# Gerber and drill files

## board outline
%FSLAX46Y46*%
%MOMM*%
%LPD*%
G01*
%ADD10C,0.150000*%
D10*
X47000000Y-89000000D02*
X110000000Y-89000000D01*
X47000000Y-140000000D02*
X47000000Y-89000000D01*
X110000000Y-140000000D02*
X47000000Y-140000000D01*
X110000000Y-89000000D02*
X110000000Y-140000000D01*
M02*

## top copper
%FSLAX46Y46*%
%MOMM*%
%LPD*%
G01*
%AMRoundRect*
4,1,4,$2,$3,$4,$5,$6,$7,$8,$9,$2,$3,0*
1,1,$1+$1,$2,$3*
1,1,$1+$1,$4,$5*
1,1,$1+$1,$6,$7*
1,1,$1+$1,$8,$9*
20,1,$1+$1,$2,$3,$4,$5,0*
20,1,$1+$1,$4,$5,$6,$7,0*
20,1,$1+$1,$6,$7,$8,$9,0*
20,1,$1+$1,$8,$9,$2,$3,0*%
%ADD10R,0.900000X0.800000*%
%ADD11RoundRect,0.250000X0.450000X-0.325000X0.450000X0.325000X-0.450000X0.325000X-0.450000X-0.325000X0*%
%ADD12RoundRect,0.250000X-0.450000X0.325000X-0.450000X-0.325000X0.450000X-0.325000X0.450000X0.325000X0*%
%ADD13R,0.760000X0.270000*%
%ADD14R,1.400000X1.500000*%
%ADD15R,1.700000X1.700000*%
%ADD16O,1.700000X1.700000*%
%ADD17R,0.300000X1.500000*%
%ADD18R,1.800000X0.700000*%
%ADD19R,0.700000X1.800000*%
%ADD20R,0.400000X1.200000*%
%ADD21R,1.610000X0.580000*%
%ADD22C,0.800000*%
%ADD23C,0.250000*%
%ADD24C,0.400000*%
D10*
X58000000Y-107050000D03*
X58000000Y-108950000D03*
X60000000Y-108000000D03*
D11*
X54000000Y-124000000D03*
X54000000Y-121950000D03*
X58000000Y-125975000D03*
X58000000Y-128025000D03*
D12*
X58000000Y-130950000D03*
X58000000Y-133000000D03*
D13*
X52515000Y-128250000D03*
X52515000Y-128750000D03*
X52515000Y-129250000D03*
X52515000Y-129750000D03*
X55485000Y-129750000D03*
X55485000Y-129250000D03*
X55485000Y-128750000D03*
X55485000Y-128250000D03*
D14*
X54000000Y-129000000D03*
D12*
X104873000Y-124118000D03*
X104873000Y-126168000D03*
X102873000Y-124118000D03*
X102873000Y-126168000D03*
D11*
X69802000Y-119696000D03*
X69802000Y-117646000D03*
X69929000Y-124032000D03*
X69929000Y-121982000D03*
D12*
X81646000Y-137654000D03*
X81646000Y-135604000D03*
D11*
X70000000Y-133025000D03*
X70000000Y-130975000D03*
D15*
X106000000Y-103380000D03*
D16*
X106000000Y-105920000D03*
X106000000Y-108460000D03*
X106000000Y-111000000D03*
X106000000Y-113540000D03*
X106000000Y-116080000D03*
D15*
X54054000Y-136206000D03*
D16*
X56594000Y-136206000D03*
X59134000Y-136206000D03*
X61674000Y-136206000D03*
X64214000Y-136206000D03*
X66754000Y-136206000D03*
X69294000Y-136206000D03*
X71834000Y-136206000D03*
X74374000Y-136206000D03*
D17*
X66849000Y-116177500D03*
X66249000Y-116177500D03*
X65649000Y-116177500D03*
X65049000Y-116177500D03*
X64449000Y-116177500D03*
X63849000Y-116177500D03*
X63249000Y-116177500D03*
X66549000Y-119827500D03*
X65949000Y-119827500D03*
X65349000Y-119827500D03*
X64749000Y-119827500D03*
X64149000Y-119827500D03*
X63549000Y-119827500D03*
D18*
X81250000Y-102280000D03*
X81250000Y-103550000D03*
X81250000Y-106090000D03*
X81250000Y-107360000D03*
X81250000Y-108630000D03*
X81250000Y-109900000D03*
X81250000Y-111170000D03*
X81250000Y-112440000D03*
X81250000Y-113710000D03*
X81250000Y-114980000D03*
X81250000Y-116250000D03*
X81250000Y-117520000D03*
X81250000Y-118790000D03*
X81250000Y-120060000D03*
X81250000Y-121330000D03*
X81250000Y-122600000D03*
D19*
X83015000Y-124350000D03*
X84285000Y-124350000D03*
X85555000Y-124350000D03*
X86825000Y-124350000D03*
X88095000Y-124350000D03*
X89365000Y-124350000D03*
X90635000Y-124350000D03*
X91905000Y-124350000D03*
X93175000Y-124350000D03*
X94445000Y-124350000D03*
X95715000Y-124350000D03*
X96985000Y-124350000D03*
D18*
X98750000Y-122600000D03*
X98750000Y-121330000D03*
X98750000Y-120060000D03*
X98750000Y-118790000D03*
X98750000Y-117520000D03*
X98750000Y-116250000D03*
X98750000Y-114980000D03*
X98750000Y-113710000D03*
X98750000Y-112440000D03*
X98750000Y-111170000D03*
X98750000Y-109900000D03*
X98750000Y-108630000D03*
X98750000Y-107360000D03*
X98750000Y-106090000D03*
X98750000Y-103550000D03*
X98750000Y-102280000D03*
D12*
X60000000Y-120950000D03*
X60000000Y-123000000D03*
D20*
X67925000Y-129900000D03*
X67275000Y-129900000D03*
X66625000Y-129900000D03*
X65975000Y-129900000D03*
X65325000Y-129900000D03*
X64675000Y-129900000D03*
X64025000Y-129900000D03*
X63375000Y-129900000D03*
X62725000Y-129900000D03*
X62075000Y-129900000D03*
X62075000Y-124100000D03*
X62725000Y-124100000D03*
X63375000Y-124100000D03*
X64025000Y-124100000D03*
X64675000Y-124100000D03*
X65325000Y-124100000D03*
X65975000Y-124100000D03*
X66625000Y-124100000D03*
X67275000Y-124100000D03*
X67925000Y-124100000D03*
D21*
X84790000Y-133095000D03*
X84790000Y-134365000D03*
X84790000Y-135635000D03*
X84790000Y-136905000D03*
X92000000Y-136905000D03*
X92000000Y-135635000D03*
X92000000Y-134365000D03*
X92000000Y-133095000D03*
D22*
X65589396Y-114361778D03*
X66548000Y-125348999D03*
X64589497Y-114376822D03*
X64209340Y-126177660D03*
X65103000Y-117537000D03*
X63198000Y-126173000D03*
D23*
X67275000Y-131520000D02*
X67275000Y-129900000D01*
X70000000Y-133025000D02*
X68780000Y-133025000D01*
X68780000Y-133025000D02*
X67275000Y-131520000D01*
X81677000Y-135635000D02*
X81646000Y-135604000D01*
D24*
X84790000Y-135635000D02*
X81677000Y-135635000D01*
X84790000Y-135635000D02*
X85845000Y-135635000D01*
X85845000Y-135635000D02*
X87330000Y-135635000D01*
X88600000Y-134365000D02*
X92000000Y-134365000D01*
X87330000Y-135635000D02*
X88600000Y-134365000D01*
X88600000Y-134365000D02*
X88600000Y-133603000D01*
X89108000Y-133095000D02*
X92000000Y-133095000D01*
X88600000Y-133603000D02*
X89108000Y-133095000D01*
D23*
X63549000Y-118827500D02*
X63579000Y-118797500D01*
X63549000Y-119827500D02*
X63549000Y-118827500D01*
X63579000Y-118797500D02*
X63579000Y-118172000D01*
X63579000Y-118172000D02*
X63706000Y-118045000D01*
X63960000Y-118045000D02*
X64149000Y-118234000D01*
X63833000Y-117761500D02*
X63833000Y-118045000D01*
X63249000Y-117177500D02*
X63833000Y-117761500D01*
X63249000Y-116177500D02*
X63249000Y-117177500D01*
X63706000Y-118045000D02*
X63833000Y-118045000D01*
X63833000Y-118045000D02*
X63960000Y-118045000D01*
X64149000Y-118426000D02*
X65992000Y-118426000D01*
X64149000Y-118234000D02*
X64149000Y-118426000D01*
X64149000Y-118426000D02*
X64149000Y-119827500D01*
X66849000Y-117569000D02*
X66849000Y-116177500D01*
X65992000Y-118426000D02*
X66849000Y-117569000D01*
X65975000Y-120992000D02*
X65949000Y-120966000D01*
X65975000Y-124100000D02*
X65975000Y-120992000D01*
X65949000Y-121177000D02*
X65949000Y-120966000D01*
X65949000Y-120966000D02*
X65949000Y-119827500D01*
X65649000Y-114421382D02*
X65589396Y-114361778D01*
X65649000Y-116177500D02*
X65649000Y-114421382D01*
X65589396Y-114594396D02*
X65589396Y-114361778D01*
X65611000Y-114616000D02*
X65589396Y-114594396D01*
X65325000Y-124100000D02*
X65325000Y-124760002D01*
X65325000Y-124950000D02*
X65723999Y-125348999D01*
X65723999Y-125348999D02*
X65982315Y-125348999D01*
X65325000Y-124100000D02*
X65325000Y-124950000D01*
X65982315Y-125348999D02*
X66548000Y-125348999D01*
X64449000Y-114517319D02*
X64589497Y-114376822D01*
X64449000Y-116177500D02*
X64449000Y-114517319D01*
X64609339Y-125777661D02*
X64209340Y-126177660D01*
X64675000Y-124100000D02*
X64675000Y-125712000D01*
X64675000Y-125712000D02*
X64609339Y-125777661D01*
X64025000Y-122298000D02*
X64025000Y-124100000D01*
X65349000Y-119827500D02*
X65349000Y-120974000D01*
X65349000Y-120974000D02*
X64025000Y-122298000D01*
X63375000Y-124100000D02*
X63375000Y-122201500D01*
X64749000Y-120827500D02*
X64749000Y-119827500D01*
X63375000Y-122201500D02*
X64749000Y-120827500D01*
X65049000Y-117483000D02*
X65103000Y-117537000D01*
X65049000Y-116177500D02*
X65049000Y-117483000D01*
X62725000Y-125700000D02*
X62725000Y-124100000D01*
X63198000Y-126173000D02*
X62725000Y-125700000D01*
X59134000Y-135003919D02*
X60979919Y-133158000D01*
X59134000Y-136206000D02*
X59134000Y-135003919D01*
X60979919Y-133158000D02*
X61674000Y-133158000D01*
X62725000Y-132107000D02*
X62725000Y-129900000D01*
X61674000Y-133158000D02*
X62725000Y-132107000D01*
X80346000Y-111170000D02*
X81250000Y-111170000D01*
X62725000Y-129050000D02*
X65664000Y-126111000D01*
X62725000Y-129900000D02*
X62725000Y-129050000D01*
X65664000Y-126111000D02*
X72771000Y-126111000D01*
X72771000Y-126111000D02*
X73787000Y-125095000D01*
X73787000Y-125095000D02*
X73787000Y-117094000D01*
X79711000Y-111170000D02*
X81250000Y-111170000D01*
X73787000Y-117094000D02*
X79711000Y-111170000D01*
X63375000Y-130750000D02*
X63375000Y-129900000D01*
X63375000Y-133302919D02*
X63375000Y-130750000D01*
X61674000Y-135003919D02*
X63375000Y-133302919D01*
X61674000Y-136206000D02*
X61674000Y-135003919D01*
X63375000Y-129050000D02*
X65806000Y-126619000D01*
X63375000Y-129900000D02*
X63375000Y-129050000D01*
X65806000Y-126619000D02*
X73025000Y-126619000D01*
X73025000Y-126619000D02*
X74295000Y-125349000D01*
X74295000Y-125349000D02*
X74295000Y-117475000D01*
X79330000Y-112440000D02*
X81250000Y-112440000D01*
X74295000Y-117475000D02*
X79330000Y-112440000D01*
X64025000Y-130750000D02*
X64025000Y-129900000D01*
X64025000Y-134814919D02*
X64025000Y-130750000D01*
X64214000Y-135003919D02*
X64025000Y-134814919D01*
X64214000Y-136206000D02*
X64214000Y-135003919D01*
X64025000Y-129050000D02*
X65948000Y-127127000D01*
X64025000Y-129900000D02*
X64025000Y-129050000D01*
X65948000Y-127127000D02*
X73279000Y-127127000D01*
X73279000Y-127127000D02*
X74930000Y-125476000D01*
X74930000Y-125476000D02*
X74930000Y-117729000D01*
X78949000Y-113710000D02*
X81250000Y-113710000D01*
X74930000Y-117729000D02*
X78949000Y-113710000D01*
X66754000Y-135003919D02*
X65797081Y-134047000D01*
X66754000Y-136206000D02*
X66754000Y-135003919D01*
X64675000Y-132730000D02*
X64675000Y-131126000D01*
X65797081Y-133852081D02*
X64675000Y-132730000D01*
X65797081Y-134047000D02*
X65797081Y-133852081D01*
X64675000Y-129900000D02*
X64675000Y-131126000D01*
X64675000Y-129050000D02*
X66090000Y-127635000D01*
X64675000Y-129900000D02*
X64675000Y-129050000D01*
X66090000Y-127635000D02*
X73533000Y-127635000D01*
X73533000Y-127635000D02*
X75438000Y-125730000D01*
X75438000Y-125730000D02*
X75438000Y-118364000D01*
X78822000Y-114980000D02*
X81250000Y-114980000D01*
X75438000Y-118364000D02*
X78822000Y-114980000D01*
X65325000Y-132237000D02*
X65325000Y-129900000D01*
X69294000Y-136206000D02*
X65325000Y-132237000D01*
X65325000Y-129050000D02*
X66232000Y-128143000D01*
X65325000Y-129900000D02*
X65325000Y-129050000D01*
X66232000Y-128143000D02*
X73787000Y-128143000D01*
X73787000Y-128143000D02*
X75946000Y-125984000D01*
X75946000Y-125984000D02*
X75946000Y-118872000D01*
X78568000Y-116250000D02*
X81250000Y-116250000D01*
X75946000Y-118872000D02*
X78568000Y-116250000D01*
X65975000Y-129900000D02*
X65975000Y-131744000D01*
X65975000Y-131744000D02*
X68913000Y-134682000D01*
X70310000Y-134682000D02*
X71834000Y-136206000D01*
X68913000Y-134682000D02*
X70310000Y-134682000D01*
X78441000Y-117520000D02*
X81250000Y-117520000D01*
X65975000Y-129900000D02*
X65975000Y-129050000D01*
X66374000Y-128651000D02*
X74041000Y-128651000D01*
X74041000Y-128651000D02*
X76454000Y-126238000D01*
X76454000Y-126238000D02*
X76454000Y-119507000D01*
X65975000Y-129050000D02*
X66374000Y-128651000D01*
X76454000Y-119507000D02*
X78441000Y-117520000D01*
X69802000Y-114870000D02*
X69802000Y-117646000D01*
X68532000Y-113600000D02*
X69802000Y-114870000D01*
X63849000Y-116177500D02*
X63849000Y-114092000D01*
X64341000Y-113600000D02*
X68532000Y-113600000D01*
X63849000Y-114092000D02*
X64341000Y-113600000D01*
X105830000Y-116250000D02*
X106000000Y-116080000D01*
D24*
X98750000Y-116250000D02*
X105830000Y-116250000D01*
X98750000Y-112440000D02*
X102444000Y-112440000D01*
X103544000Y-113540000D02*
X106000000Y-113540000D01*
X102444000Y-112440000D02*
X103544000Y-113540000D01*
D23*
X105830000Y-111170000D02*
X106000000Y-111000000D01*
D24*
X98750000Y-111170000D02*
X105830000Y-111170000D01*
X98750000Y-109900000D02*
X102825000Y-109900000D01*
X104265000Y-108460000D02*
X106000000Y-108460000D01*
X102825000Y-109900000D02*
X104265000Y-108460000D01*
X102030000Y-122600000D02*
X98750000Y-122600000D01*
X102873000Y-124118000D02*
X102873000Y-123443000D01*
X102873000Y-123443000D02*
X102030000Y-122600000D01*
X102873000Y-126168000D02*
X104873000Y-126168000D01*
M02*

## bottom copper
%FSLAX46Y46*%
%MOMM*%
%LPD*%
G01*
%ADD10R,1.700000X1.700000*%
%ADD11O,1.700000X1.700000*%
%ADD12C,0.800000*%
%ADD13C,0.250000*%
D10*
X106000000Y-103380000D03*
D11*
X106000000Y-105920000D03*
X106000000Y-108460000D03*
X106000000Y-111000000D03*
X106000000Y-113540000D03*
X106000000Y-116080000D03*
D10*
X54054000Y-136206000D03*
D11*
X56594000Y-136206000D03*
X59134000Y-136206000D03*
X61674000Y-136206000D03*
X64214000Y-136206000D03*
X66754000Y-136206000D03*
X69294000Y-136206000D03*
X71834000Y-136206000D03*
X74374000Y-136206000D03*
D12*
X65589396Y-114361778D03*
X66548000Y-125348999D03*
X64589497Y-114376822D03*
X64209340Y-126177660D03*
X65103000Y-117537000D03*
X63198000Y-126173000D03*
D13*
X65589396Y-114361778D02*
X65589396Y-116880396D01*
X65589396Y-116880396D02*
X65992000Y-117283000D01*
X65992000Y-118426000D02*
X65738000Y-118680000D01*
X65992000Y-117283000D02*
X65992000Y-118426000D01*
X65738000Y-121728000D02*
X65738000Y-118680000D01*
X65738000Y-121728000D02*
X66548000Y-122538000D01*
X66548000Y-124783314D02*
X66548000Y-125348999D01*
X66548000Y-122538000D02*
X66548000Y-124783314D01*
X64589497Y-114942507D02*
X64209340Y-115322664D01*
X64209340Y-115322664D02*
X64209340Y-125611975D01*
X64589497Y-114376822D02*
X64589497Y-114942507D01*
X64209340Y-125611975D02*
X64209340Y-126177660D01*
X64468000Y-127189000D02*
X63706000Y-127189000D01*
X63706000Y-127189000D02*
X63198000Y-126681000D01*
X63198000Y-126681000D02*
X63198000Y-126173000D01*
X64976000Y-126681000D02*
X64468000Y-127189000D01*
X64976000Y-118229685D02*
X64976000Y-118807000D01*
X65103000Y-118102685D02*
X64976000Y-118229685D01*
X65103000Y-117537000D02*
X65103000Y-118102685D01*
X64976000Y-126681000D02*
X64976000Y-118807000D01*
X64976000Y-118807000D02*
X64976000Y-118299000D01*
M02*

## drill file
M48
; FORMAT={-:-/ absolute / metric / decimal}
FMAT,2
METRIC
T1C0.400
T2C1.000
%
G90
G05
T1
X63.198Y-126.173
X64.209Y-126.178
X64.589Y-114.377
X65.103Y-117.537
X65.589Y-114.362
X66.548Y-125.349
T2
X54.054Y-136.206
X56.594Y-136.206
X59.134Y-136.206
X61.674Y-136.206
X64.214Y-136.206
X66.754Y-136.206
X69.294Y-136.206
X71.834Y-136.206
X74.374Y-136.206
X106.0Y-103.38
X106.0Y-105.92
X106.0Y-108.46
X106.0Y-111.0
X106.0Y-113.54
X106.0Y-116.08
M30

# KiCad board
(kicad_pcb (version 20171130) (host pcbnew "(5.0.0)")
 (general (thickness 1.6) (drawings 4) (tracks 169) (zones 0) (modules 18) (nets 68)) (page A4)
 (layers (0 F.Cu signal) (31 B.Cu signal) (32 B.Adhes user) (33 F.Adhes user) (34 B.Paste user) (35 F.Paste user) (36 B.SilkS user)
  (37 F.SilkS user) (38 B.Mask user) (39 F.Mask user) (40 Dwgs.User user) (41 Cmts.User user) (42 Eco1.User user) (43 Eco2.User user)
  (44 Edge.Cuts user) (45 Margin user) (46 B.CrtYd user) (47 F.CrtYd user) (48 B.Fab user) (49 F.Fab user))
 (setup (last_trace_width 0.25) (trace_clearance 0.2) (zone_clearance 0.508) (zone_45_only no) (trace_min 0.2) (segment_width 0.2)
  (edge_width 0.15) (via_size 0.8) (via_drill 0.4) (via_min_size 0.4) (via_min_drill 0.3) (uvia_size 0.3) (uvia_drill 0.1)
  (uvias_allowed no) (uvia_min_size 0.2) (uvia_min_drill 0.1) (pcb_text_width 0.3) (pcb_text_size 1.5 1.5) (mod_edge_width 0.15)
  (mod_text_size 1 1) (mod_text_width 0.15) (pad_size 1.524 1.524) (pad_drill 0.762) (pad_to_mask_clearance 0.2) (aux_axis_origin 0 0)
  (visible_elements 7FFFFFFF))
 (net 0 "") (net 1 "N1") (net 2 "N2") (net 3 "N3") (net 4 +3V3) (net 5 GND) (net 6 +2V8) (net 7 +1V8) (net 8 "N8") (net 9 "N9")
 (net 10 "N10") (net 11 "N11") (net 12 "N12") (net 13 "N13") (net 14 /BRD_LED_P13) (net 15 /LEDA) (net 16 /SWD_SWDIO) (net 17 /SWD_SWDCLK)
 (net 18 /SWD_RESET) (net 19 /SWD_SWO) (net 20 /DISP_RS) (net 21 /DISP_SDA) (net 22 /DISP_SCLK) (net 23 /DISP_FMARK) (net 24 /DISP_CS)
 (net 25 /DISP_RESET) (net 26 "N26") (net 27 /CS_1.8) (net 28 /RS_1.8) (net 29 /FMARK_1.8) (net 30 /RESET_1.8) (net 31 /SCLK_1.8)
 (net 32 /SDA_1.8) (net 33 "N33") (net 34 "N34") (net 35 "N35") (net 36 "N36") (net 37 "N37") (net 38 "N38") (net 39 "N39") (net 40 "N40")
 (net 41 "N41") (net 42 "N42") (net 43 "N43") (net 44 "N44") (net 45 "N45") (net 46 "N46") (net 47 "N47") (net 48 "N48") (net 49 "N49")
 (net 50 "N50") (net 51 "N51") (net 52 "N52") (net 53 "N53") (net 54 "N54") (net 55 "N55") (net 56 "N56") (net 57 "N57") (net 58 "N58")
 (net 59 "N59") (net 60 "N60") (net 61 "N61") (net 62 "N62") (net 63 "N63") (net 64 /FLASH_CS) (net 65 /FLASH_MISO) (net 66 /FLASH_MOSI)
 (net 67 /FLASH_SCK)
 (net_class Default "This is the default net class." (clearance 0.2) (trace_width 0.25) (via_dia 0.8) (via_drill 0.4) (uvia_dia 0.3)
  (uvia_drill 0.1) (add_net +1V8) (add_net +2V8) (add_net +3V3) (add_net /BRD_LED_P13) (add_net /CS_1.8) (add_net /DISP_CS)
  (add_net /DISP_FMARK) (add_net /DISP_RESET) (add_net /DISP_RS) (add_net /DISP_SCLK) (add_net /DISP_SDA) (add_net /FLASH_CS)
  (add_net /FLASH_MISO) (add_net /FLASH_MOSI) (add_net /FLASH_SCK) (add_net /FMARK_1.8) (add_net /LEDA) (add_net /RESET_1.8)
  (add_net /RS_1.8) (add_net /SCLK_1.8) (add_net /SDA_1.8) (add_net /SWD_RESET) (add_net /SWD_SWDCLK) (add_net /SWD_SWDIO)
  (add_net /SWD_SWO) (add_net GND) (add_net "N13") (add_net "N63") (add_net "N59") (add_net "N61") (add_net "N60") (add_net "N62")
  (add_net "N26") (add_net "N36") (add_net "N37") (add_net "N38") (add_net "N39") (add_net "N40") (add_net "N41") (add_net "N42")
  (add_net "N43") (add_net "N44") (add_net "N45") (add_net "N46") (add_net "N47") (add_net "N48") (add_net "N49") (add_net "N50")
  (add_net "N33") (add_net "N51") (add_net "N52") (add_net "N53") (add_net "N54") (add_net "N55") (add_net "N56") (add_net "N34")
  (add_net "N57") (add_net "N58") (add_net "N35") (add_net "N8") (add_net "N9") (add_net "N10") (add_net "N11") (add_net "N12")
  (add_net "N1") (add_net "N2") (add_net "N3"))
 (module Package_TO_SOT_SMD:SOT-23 (layer F.Cu) (at 59 108)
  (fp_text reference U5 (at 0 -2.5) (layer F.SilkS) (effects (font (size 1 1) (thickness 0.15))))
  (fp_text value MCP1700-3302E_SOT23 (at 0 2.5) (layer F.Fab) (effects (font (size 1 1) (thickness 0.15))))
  (pad 1 smd rect (at -1 -0.95) (size 0.9 0.8) (layers F.Cu F.Paste F.Mask) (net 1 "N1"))
  (pad 2 smd rect (at -1 0.95) (size 0.9 0.8) (layers F.Cu F.Paste F.Mask) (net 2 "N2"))
  (pad 3 smd rect (at 1 0) (size 0.9 0.8) (layers F.Cu F.Paste F.Mask) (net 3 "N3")))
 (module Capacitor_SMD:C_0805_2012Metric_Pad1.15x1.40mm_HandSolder (layer F.Cu) (at 54 122.975 90)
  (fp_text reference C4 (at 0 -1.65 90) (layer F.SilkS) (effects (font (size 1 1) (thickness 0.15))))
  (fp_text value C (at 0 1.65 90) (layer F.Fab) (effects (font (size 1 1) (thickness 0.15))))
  (pad 1 smd roundrect (at -1.025 0 90) (size 1.15 1.4) (layers F.Cu F.Paste F.Mask) (roundrect_rratio 0.217391) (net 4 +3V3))
  (pad 2 smd roundrect (at 1.025 0 90) (size 1.15 1.4) (layers F.Cu F.Paste F.Mask) (roundrect_rratio 0.217391) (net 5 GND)))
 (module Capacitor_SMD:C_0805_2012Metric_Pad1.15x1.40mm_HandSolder (layer F.Cu) (at 58 127 90)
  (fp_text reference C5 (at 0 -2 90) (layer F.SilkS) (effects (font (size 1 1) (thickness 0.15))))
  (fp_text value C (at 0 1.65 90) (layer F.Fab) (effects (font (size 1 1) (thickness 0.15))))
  (pad 2 smd roundrect (at 1.025 0 90) (size 1.15 1.4) (layers F.Cu F.Paste F.Mask) (roundrect_rratio 0.217391) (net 5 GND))
  (pad 1 smd roundrect (at -1.025 0 90) (size 1.15 1.4) (layers F.Cu F.Paste F.Mask) (roundrect_rratio 0.217391) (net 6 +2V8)))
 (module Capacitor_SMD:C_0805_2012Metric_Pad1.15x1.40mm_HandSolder (layer F.Cu) (at 58 131.975 270)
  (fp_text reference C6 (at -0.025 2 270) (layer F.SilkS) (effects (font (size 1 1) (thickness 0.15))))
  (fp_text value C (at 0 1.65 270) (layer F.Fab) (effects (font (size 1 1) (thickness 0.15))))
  (pad 1 smd roundrect (at -1.025 0 270) (size 1.15 1.4) (layers F.Cu F.Paste F.Mask) (roundrect_rratio 0.217391) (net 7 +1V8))
  (pad 2 smd roundrect (at 1.025 0 270) (size 1.15 1.4) (layers F.Cu F.Paste F.Mask) (roundrect_rratio 0.217391) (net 5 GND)))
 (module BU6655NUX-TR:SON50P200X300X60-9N (layer F.Cu) (at 54 129)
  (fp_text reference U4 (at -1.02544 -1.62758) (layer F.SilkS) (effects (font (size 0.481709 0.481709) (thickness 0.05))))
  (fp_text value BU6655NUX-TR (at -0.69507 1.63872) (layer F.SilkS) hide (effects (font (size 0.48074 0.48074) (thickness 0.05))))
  (pad 1 smd rect (at -1.485 -0.75) (size 0.76 0.27) (layers F.Cu F.Paste F.Mask) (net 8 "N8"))
  (pad 2 smd rect (at -1.485 -0.25) (size 0.76 0.27) (layers F.Cu F.Paste F.Mask) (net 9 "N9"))
  (pad 3 smd rect (at -1.485 0.25) (size 0.76 0.27) (layers F.Cu F.Paste F.Mask) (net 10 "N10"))
  (pad 4 smd rect (at -1.485 0.75) (size 0.76 0.27) (layers F.Cu F.Paste F.Mask) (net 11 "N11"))
  (pad 5 smd rect (at 1.485 0.75) (size 0.76 0.27) (layers F.Cu F.Paste F.Mask) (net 5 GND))
  (pad 6 smd rect (at 1.485 0.25) (size 0.76 0.27) (layers F.Cu F.Paste F.Mask) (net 7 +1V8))
  (pad 7 smd rect (at 1.485 -0.25) (size 0.76 0.27) (layers F.Cu F.Paste F.Mask) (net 6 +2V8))
  (pad 8 smd rect (at 1.485 -0.75) (size 0.76 0.27) (layers F.Cu F.Paste F.Mask) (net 4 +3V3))
  (pad 9 smd rect (at 0 0) (size 1.4 1.5) (layers F.Cu F.Paste F.Mask) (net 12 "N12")))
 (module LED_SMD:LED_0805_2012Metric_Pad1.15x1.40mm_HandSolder (layer F.Cu) (at 104.873 125.143 270)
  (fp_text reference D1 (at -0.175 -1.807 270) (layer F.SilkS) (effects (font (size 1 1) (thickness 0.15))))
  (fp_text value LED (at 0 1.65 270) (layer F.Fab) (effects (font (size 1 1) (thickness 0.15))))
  (pad 1 smd roundrect (at -1.025 0 270) (size 1.15 1.4) (layers F.Cu F.Paste F.Mask) (roundrect_rratio 0.217391) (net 5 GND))
  (pad 2 smd roundrect (at 1.025 0 270) (size 1.15 1.4) (layers F.Cu F.Paste F.Mask) (roundrect_rratio 0.217391) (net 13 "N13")))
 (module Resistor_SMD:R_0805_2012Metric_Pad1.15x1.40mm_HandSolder (layer F.Cu) (at 102.873 125.143 270)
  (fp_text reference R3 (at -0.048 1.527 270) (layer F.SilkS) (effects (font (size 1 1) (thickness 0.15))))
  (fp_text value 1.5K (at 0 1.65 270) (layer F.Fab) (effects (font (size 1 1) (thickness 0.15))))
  (pad 1 smd roundrect (at -1.025 0 270) (size 1.15 1.4) (layers F.Cu F.Paste F.Mask) (roundrect_rratio 0.217391) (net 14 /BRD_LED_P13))
  (pad 2 smd roundrect (at 1.025 0 270) (size 1.15 1.4) (layers F.Cu F.Paste F.Mask) (roundrect_rratio 0.217391) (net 13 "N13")))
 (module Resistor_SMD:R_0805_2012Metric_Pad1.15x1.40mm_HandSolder (layer F.Cu) (at 69.802 118.671 90)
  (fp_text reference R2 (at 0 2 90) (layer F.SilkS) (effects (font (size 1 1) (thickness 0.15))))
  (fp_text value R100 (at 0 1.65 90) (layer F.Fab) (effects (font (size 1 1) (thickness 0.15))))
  (pad 1 smd roundrect (at -1.025 0 90) (size 1.15 1.4) (layers F.Cu F.Paste F.Mask) (roundrect_rratio 0.217391) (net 4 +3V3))
  (pad 2 smd roundrect (at 1.025 0 90) (size 1.15 1.4) (layers F.Cu F.Paste F.Mask) (roundrect_rratio 0.217391) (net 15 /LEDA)))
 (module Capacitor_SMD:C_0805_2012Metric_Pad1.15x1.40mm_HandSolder (layer F.Cu) (at 69.929 123.007 90)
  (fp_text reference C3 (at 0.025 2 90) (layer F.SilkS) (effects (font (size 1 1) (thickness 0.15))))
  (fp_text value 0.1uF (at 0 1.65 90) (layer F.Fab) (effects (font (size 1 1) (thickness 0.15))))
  (pad 1 smd roundrect (at -1.025 0 90) (size 1.15 1.4) (layers F.Cu F.Paste F.Mask) (roundrect_rratio 0.217391) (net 7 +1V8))
  (pad 2 smd roundrect (at 1.025 0 90) (size 1.15 1.4) (layers F.Cu F.Paste F.Mask) (roundrect_rratio 0.217391) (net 5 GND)))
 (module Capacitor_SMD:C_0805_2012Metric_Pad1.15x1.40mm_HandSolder (layer F.Cu) (at 81.646 136.629 270)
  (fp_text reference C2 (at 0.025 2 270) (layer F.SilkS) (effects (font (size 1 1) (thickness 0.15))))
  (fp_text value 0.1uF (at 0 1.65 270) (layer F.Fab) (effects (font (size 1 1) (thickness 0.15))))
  (pad 2 smd roundrect (at 1.025 0 270) (size 1.15 1.4) (layers F.Cu F.Paste F.Mask) (roundrect_rratio 0.217391) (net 5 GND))
  (pad 1 smd roundrect (at -1.025 0 270) (size 1.15 1.4) (layers F.Cu F.Paste F.Mask) (roundrect_rratio 0.217391) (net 4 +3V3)))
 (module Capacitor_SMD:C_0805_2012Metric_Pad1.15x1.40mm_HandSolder (layer F.Cu) (at 70 132 90)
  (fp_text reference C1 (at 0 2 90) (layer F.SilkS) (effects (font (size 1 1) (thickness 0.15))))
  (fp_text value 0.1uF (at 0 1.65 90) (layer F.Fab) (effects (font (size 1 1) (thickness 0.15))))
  (pad 1 smd roundrect (at -1.025 0 90) (size 1.15 1.4) (layers F.Cu F.Paste F.Mask) (roundrect_rratio 0.217391) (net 4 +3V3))
  (pad 2 smd roundrect (at 1.025 0 90) (size 1.15 1.4) (layers F.Cu F.Paste F.Mask) (roundrect_rratio 0.217391) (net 5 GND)))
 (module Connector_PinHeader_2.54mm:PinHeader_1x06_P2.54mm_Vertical (layer F.Cu) (at 106 103.38)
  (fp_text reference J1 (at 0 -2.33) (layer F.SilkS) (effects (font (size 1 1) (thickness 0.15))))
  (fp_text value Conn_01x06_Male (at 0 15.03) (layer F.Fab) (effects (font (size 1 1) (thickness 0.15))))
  (pad 1 thru_hole rect (at 0 0) (size 1.7 1.7) (drill 1) (layers *.Cu *.Mask) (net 4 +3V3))
  (pad 2 thru_hole oval (at 0 2.54) (size 1.7 1.7) (drill 1) (layers *.Cu *.Mask) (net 5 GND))
  (pad 3 thru_hole oval (at 0 5.08) (size 1.7 1.7) (drill 1) (layers *.Cu *.Mask) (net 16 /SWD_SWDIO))
  (pad 4 thru_hole oval (at 0 7.62) (size 1.7 1.7) (drill 1) (layers *.Cu *.Mask) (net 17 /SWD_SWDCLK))
  (pad 5 thru_hole oval (at 0 10.16) (size 1.7 1.7) (drill 1) (layers *.Cu *.Mask) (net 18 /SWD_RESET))
  (pad 6 thru_hole oval (at 0 12.7) (size 1.7 1.7) (drill 1) (layers *.Cu *.Mask) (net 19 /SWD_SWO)))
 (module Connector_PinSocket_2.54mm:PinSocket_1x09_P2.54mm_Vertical (layer F.Cu) (at 54.054 136.206 90)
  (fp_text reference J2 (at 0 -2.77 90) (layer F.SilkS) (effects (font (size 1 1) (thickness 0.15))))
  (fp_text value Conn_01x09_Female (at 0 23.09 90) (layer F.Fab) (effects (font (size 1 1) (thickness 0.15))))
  (pad 1 thru_hole rect (at 0 0 90) (size 1.7 1.7) (drill 1) (layers *.Cu *.Mask) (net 4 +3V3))
  (pad 2 thru_hole oval (at 0 2.54 90) (size 1.7 1.7) (drill 1) (layers *.Cu *.Mask) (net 5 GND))
  (pad 3 thru_hole oval (at 0 5.08 90) (size 1.7 1.7) (drill 1) (layers *.Cu *.Mask) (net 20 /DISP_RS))
  (pad 4 thru_hole oval (at 0 7.62 90) (size 1.7 1.7) (drill 1) (layers *.Cu *.Mask) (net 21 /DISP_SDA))
  (pad 5 thru_hole oval (at 0 10.16 90) (size 1.7 1.7) (drill 1) (layers *.Cu *.Mask) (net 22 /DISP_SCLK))
  (pad 6 thru_hole oval (at 0 12.7 90) (size 1.7 1.7) (drill 1) (layers *.Cu *.Mask) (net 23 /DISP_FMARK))
  (pad 7 thru_hole oval (at 0 15.24 90) (size 1.7 1.7) (drill 1) (layers *.Cu *.Mask) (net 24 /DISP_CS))
  (pad 8 thru_hole oval (at 0 17.78 90) (size 1.7 1.7) (drill 1) (layers *.Cu *.Mask) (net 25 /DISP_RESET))
  (pad 9 thru_hole oval (at 0 20.32 90) (size 1.7 1.7) (drill 1) (layers *.Cu *.Mask) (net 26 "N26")))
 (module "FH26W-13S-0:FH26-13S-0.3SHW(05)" (layer F.Cu) (at 64.849 117.7275)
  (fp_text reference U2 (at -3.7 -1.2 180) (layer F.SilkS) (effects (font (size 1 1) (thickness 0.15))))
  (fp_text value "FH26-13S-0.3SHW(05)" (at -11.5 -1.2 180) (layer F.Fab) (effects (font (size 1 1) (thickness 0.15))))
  (pad 13 smd rect (at 2 -1.55 180) (size 0.3 1.5) (layers F.Cu F.Paste F.Mask) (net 5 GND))
  (pad 11 smd rect (at 1.4 -1.55 180) (size 0.3 1.5) (layers F.Cu F.Paste F.Mask) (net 7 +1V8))
  (pad 9 smd rect (at 0.8 -1.55 180) (size 0.3 1.5) (layers F.Cu F.Paste F.Mask) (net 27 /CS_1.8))
  (pad 7 smd rect (at 0.2 -1.55 180) (size 0.3 1.5) (layers F.Cu F.Paste F.Mask) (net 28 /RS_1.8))
  (pad 5 smd rect (at -0.4 -1.55 180) (size 0.3 1.5) (layers F.Cu F.Paste F.Mask) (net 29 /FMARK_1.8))
  (pad 3 smd rect (at -1 -1.55 180) (size 0.3 1.5) (layers F.Cu F.Paste F.Mask) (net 15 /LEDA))
  (pad 1 smd rect (at -1.6 -1.55 180) (size 0.3 1.5) (layers F.Cu F.Paste F.Mask) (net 5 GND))
  (pad 12 smd rect (at 1.7 2.1 180) (size 0.3 1.5) (layers F.Cu F.Paste F.Mask) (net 6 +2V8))
  (pad 10 smd rect (at 1.1 2.1 180) (size 0.3 1.5) (layers F.Cu F.Paste F.Mask) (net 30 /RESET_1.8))
  (pad 8 smd rect (at 0.5 2.1 180) (size 0.3 1.5) (layers F.Cu F.Paste F.Mask) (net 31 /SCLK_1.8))
  (pad 6 smd rect (at -0.1 2.1 180) (size 0.3 1.5) (layers F.Cu F.Paste F.Mask) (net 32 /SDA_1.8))
  (pad 4 smd rect (at -0.7 2.1 180) (size 0.3 1.5) (layers F.Cu F.Paste F.Mask) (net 5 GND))
  (pad 2 smd rect (at -1.3 2.1 180) (size 0.3 1.5) (layers F.Cu F.Paste F.Mask) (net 5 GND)))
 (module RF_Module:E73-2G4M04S (layer F.Cu) (at 90 110)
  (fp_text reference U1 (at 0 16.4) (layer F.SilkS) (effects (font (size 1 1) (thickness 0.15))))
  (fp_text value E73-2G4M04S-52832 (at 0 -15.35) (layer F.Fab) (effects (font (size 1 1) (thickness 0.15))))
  (pad 0 smd rect (at -8.75 -7.72) (size 1.8 0.7) (layers F.Cu F.Paste F.Mask) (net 5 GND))
  (pad 1 smd rect (at -8.75 -6.45) (size 1.8 0.7) (layers F.Cu F.Paste F.Mask) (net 5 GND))
  (pad 2 smd rect (at -8.75 -3.91) (size 1.8 0.7) (layers F.Cu F.Paste F.Mask) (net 5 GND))
  (pad 3 smd rect (at -8.75 -2.64) (size 1.8 0.7) (layers F.Cu F.Paste F.Mask) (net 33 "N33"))
  (pad 4 smd rect (at -8.75 -1.37) (size 1.8 0.7) (layers F.Cu F.Paste F.Mask) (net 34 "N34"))
  (pad 5 smd rect (at -8.75 -0.1) (size 1.8 0.7) (layers F.Cu F.Paste F.Mask) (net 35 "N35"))
  (pad 6 smd rect (at -8.75 1.17) (size 1.8 0.7) (layers F.Cu F.Paste F.Mask) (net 20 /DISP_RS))
  (pad 7 smd rect (at -8.75 2.44) (size 1.8 0.7) (layers F.Cu F.Paste F.Mask) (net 21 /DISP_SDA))
  (pad 8 smd rect (at -8.75 3.71) (size 1.8 0.7) (layers F.Cu F.Paste F.Mask) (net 22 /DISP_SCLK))
  (pad 9 smd rect (at -8.75 4.98) (size 1.8 0.7) (layers F.Cu F.Paste F.Mask) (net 23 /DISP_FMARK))
  (pad 10 smd rect (at -8.75 6.25) (size 1.8 0.7) (layers F.Cu F.Paste F.Mask) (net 24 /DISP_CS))
  (pad 11 smd rect (at -8.75 7.52) (size 1.8 0.7) (layers F.Cu F.Paste F.Mask) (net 25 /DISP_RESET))
  (pad 12 smd rect (at -8.75 8.79) (size 1.8 0.7) (layers F.Cu F.Paste F.Mask) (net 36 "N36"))
  (pad 13 smd rect (at -8.75 10.06) (size 1.8 0.7) (layers F.Cu F.Paste F.Mask) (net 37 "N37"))
  (pad 14 smd rect (at -8.75 11.33) (size 1.8 0.7) (layers F.Cu F.Paste F.Mask) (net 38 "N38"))
  (pad 15 smd rect (at -8.75 12.6) (size 1.8 0.7) (layers F.Cu F.Paste F.Mask) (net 5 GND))
  (pad 16 smd rect (at -6.985 14.35) (size 0.7 1.8) (layers F.Cu F.Paste F.Mask) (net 4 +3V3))
  (pad 17 smd rect (at -5.715 14.35) (size 0.7 1.8) (layers F.Cu F.Paste F.Mask) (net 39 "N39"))
  (pad 18 smd rect (at -4.445 14.35) (size 0.7 1.8) (layers F.Cu F.Paste F.Mask) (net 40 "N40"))
  (pad 19 smd rect (at -3.175 14.35) (size 0.7 1.8) (layers F.Cu F.Paste F.Mask) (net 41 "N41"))
  (pad 20 smd rect (at -1.905 14.35) (size 0.7 1.8) (layers F.Cu F.Paste F.Mask) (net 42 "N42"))
  (pad 21 smd rect (at -0.635 14.35) (size 0.7 1.8) (layers F.Cu F.Paste F.Mask) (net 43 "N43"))
  (pad 22 smd rect (at 0.635 14.35) (size 0.7 1.8) (layers F.Cu F.Paste F.Mask) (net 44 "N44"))
  (pad 23 smd rect (at 1.905 14.35) (size 0.7 1.8) (layers F.Cu F.Paste F.Mask) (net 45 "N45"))
  (pad 24 smd rect (at 3.175 14.35) (size 0.7 1.8) (layers F.Cu F.Paste F.Mask) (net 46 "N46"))
  (pad 25 smd rect (at 4.445 14.35) (size 0.7 1.8) (layers F.Cu F.Paste F.Mask) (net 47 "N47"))
  (pad 26 smd rect (at 5.715 14.35) (size 0.7 1.8) (layers F.Cu F.Paste F.Mask) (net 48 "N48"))
  (pad 27 smd rect (at 6.985 14.35) (size 0.7 1.8) (layers F.Cu F.Paste F.Mask) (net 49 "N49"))
  (pad 28 smd rect (at 8.75 12.6) (size 1.8 0.7) (layers F.Cu F.Paste F.Mask) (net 14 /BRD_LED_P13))
  (pad 29 smd rect (at 8.75 11.33) (size 1.8 0.7) (layers F.Cu F.Paste F.Mask) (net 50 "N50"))
  (pad 30 smd rect (at 8.75 10.06) (size 1.8 0.7) (layers F.Cu F.Paste F.Mask) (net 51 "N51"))
  (pad 31 smd rect (at 8.75 8.79) (size 1.8 0.7) (layers F.Cu F.Paste F.Mask) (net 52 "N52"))
  (pad 32 smd rect (at 8.75 7.52) (size 1.8 0.7) (layers F.Cu F.Paste F.Mask) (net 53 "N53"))
  (pad 33 smd rect (at 8.75 6.25) (size 1.8 0.7) (layers F.Cu F.Paste F.Mask) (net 19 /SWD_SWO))
  (pad 34 smd rect (at 8.75 4.98) (size 1.8 0.7) (layers F.Cu F.Paste F.Mask) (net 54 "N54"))
  (pad 35 smd rect (at 8.75 3.71) (size 1.8 0.7) (layers F.Cu F.Paste F.Mask) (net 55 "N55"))
  (pad 36 smd rect (at 8.75 2.44) (size 1.8 0.7) (layers F.Cu F.Paste F.Mask) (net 18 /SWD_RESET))
  (pad 37 smd rect (at 8.75 1.17) (size 1.8 0.7) (layers F.Cu F.Paste F.Mask) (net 17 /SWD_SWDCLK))
  (pad 38 smd rect (at 8.75 -0.1) (size 1.8 0.7) (layers F.Cu F.Paste F.Mask) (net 16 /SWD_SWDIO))
  (pad 39 smd rect (at 8.75 -1.37) (size 1.8 0.7) (layers F.Cu F.Paste F.Mask) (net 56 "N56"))
  (pad 40 smd rect (at 8.75 -2.64) (size 1.8 0.7) (layers F.Cu F.Paste F.Mask) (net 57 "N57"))
  (pad 41 smd rect (at 8.75 -3.91) (size 1.8 0.7) (layers F.Cu F.Paste F.Mask) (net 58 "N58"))
  (pad 42 smd rect (at 8.75 -6.45) (size 1.8 0.7) (layers F.Cu F.Paste F.Mask) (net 5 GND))
  (pad 43 smd rect (at 8.75 -7.72) (size 1.8 0.7) (layers F.Cu F.Paste F.Mask) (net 5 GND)))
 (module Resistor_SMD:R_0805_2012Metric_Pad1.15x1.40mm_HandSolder (layer F.Cu) (at 60 121.975 270)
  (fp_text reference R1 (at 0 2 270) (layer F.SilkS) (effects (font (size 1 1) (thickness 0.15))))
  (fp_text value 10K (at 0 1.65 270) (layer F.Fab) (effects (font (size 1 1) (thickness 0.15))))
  (pad 1 smd roundrect (at -1.025 0 270) (size 1.15 1.4) (layers F.Cu F.Paste F.Mask) (roundrect_rratio 0.217391) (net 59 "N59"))
  (pad 2 smd roundrect (at 1.025 0 270) (size 1.15 1.4) (layers F.Cu F.Paste F.Mask) (roundrect_rratio 0.217391) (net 7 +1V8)))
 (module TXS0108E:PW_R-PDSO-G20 (layer F.Cu) (at 65 127 180)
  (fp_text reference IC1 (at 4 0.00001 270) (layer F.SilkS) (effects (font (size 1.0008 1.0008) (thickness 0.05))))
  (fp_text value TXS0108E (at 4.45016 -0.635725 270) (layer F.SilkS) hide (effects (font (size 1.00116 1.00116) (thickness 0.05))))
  (pad 20 smd rect (at -2.925 -2.9) (size 0.4 1.2) (layers F.Cu F.Paste F.Mask) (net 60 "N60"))
  (pad 19 smd rect (at -2.275 -2.9) (size 0.4 1.2) (layers F.Cu F.Paste F.Mask) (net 4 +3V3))
  (pad 18 smd rect (at -1.625 -2.9) (size 0.4 1.2) (layers F.Cu F.Paste F.Mask) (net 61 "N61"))
  (pad 17 smd rect (at -0.975 -2.9) (size 0.4 1.2) (layers F.Cu F.Paste F.Mask) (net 25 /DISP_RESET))
  (pad 16 smd rect (at -0.325 -2.9) (size 0.4 1.2) (layers F.Cu F.Paste F.Mask) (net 24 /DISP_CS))
  (pad 15 smd rect (at 0.325 -2.9) (size 0.4 1.2) (layers F.Cu F.Paste F.Mask) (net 23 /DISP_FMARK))
  (pad 14 smd rect (at 0.975 -2.9) (size 0.4 1.2) (layers F.Cu F.Paste F.Mask) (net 22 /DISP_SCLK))
  (pad 13 smd rect (at 1.625 -2.9) (size 0.4 1.2) (layers F.Cu F.Paste F.Mask) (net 21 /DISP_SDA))
  (pad 12 smd rect (at 2.275 -2.9) (size 0.4 1.2) (layers F.Cu F.Paste F.Mask) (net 20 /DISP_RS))
  (pad 11 smd rect (at 2.925 -2.9) (size 0.4 1.2) (layers F.Cu F.Paste F.Mask) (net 5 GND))
  (pad 10 smd rect (at 2.925 2.9 180) (size 0.4 1.2) (layers F.Cu F.Paste F.Mask) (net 59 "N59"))
  (pad 9 smd rect (at 2.275 2.9 180) (size 0.4 1.2) (layers F.Cu F.Paste F.Mask) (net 28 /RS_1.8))
  (pad 8 smd rect (at 1.625 2.9 180) (size 0.4 1.2) (layers F.Cu F.Paste F.Mask) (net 32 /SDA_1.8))
  (pad 7 smd rect (at 0.975 2.9 180) (size 0.4 1.2) (layers F.Cu F.Paste F.Mask) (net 31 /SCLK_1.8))
  (pad 6 smd rect (at 0.325 2.9 180) (size 0.4 1.2) (layers F.Cu F.Paste F.Mask) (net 29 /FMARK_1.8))
  (pad 5 smd rect (at -0.325 2.9 180) (size 0.4 1.2) (layers F.Cu F.Paste F.Mask) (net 27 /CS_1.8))
  (pad 4 smd rect (at -0.975 2.9 180) (size 0.4 1.2) (layers F.Cu F.Paste F.Mask) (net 30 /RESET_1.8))
  (pad 3 smd rect (at -1.625 2.9 180) (size 0.4 1.2) (layers F.Cu F.Paste F.Mask) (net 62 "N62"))
  (pad 2 smd rect (at -2.275 2.9 180) (size 0.4 1.2) (layers F.Cu F.Paste F.Mask) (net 7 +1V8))
  (pad 1 smd rect (at -2.925 2.9 180) (size 0.4 1.2) (layers F.Cu F.Paste F.Mask) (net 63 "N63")))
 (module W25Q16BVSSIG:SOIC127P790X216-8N (layer F.Cu) (at 88.395 135)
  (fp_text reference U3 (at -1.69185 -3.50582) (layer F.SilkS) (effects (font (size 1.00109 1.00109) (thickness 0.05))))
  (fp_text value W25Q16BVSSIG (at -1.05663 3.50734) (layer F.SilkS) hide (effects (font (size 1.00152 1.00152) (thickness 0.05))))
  (pad 1 smd rect (at -3.605 -1.905) (size 1.61 0.58) (layers F.Cu F.Paste F.Mask) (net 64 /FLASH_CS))
  (pad 2 smd rect (at -3.605 -0.635) (size 1.61 0.58) (layers F.Cu F.Paste F.Mask) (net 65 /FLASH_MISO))
  (pad 3 smd rect (at -3.605 0.635) (size 1.61 0.58) (layers F.Cu F.Paste F.Mask) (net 4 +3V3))
  (pad 4 smd rect (at -3.605 1.905) (size 1.61 0.58) (layers F.Cu F.Paste F.Mask) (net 5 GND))
  (pad 5 smd rect (at 3.605 1.905) (size 1.61 0.58) (layers F.Cu F.Paste F.Mask) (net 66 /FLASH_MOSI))
  (pad 6 smd rect (at 3.605 0.635) (size 1.61 0.58) (layers F.Cu F.Paste F.Mask) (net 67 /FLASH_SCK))
  (pad 7 smd rect (at 3.605 -0.635) (size 1.61 0.58) (layers F.Cu F.Paste F.Mask) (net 4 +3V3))
  (pad 8 smd rect (at 3.605 -1.905) (size 1.61 0.58) (layers F.Cu F.Paste F.Mask) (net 4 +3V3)))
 (gr_line (start 47 89) (end 110 89) (layer Edge.Cuts) (width 0.15))
 (gr_line (start 47 140) (end 47 89) (layer Edge.Cuts) (width 0.15))
 (gr_line (start 110 140) (end 47 140) (layer Edge.Cuts) (width 0.15))
 (gr_line (start 110 89) (end 110 140) (layer Edge.Cuts) (width 0.15))
 (segment (start 67.275 131.52) (end 67.275 129.9) (width 0.25) (layer F.Cu) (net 4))
 (segment (start 70 133.025) (end 68.78 133.025) (width 0.25) (layer F.Cu) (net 4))
 (segment (start 68.78 133.025) (end 67.275 131.52) (width 0.25) (layer F.Cu) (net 4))
 (segment (start 81.677 135.635) (end 81.646 135.604) (width 0.25) (layer F.Cu) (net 4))
 (segment (start 84.79 135.635) (end 81.677 135.635) (width 0.4) (layer F.Cu) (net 4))
 (segment (start 84.79 135.635) (end 85.845 135.635) (width 0.4) (layer F.Cu) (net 4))
 (segment (start 85.845 135.635) (end 87.33 135.635) (width 0.4) (layer F.Cu) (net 4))
 (segment (start 88.6 134.365) (end 92 134.365) (width 0.4) (layer F.Cu) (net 4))
 (segment (start 87.33 135.635) (end 88.6 134.365) (width 0.4) (layer F.Cu) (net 4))
 (segment (start 88.6 134.365) (end 88.6 133.603) (width 0.4) (layer F.Cu) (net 4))
 (segment (start 89.108 133.095) (end 92 133.095) (width 0.4) (layer F.Cu) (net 4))
 (segment (start 88.6 133.603) (end 89.108 133.095) (width 0.4) (layer F.Cu) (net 4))
 (segment (start 63.549 118.8275) (end 63.579 118.7975) (width 0.25) (layer F.Cu) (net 5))
 (segment (start 63.549 119.8275) (end 63.549 118.8275) (width 0.25) (layer F.Cu) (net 5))
 (segment (start 63.579 118.7975) (end 63.579 118.172) (width 0.25) (layer F.Cu) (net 5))
 (segment (start 63.579 118.172) (end 63.706 118.045) (width 0.25) (layer F.Cu) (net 5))
 (segment (start 63.96 118.045) (end 64.149 118.234) (width 0.25) (layer F.Cu) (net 5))
 (segment (start 63.833 117.7615) (end 63.833 118.045) (width 0.25) (layer F.Cu) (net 5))
 (segment (start 63.249 117.1775) (end 63.833 117.7615) (width 0.25) (layer F.Cu) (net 5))
 (segment (start 63.249 116.1775) (end 63.249 117.1775) (width 0.25) (layer F.Cu) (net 5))
 (segment (start 63.706 118.045) (end 63.833 118.045) (width 0.25) (layer F.Cu) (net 5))
 (segment (start 63.833 118.045) (end 63.96 118.045) (width 0.25) (layer F.Cu) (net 5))
 (segment (start 64.149 118.426) (end 65.992 118.426) (width 0.25) (layer F.Cu) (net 5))
 (segment (start 64.149 118.234) (end 64.149 118.426) (width 0.25) (layer F.Cu) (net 5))
 (segment (start 64.149 118.426) (end 64.149 119.8275) (width 0.25) (layer F.Cu) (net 5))
 (segment (start 66.849 117.569) (end 66.849 116.1775) (width 0.25) (layer F.Cu) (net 5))
 (segment (start 65.992 118.426) (end 66.849 117.569) (width 0.25) (layer F.Cu) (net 5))
 (segment (start 65.975 120.992) (end 65.949 120.966) (width 0.25) (layer F.Cu) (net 30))
 (segment (start 65.975 124.1) (end 65.975 120.992) (width 0.25) (layer F.Cu) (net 30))
 (segment (start 65.949 121.177) (end 65.949 120.966) (width 0.25) (layer F.Cu) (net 30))
 (segment (start 65.949 120.966) (end 65.949 119.8275) (width 0.25) (layer F.Cu) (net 30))
 (via (at 65.589396 114.361778) (size 0.8) (drill 0.4) (layers F.Cu B.Cu) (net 27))
 (segment (start 65.649 114.421382) (end 65.589396 114.361778) (width 0.25) (layer F.Cu) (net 27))
 (segment (start 65.649 116.1775) (end 65.649 114.421382) (width 0.25) (layer F.Cu) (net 27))
 (segment (start 65.589396 114.594396) (end 65.589396 114.361778) (width 0.25) (layer F.Cu) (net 27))
 (segment (start 65.611 114.616) (end 65.589396 114.594396) (width 0.25) (layer F.Cu) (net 27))
 (segment (start 65.589396 114.361778) (end 65.589396 116.880396) (width 0.25) (layer B.Cu) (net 27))
 (segment (start 65.589396 116.880396) (end 65.992 117.283) (width 0.25) (layer B.Cu) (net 27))
 (segment (start 65.992 118.426) (end 65.738 118.68) (width 0.25) (layer B.Cu) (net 27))
 (segment (start 65.992 117.283) (end 65.992 118.426) (width 0.25) (layer B.Cu) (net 27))
 (segment (start 65.325 124.1) (end 65.325 124.760002) (width 0.25) (layer F.Cu) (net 27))
 (segment (start 65.738 121.728) (end 65.738 118.68) (width 0.25) (layer B.Cu) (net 27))
 (via (at 66.548 125.348999) (size 0.8) (drill 0.4) (layers F.Cu B.Cu) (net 27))
 (segment (start 65.738 121.728) (end 66.548 122.538) (width 0.25) (layer B.Cu) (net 27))
 (segment (start 65.325 124.95) (end 65.723999 125.348999) (width 0.25) (layer F.Cu) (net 27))
 (segment (start 65.723999 125.348999) (end 65.982315 125.348999) (width 0.25) (layer F.Cu) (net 27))
 (segment (start 65.325 124.1) (end 65.325 124.95) (width 0.25) (layer F.Cu) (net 27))
 (segment (start 66.548 124.783314) (end 66.548 125.348999) (width 0.25) (layer B.Cu) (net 27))
 (segment (start 65.982315 125.348999) (end 66.548 125.348999) (width 0.25) (layer F.Cu) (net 27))
 (segment (start 66.548 122.538) (end 66.548 124.783314) (width 0.25) (layer B.Cu) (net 27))
 (via (at 64.589497 114.376822) (size 0.8) (drill 0.4) (layers F.Cu B.Cu) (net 29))
 (segment (start 64.449 114.517319) (end 64.589497 114.376822) (width 0.25) (layer F.Cu) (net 29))
 (segment (start 64.449 116.1775) (end 64.449 114.517319) (width 0.25) (layer F.Cu) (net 29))
 (via (at 64.20934 126.17766) (size 0.8) (drill 0.4) (layers F.Cu B.Cu) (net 29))
 (segment (start 64.589497 114.942507) (end 64.20934 115.322664) (width 0.25) (layer B.Cu) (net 29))
 (segment (start 64.20934 115.322664) (end 64.20934 125.611975) (width 0.25) (layer B.Cu) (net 29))
 (segment (start 64.589497 114.376822) (end 64.589497 114.942507) (width 0.25) (layer B.Cu) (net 29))
 (segment (start 64.609339 125.777661) (end 64.20934 126.17766) (width 0.25) (layer F.Cu) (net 29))
 (segment (start 64.20934 125.611975) (end 64.20934 126.17766) (width 0.25) (layer B.Cu) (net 29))
 (segment (start 64.675 124.1) (end 64.675 125.712) (width 0.25) (layer F.Cu) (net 29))
 (segment (start 64.675 125.712) (end 64.609339 125.777661) (width 0.25) (layer F.Cu) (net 29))
 (segment (start 64.025 122.298) (end 64.025 124.1) (width 0.25) (layer F.Cu) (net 31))
 (segment (start 65.349 119.8275) (end 65.349 120.974) (width 0.25) (layer F.Cu) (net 31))
 (segment (start 65.349 120.974) (end 64.025 122.298) (width 0.25) (layer F.Cu) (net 31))
 (segment (start 63.375 124.1) (end 63.375 122.2015) (width 0.25) (layer F.Cu) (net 32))
 (segment (start 64.749 120.8275) (end 64.749 119.8275) (width 0.25) (layer F.Cu) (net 32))
 (segment (start 63.375 122.2015) (end 64.749 120.8275) (width 0.25) (layer F.Cu) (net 32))
 (via (at 65.103 117.537) (size 0.8) (drill 0.4) (layers F.Cu B.Cu) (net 28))
 (segment (start 65.049 117.483) (end 65.103 117.537) (width 0.25) (layer F.Cu) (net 28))
 (segment (start 65.049 116.1775) (end 65.049 117.483) (width 0.25) (layer F.Cu) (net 28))
 (segment (start 64.468 127.189) (end 63.706 127.189) (width 0.25) (layer B.Cu) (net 28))
 (via (at 63.198 126.173) (size 0.8) (drill 0.4) (layers F.Cu B.Cu) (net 28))
 (segment (start 63.706 127.189) (end 63.198 126.681) (width 0.25) (layer B.Cu) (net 28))
 (segment (start 63.198 126.681) (end 63.198 126.173) (width 0.25) (layer B.Cu) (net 28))
 (segment (start 62.725 125.7) (end 62.725 124.1) (width 0.25) (layer F.Cu) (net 28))
 (segment (start 63.198 126.173) (end 62.725 125.7) (width 0.25) (layer F.Cu) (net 28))
 (segment (start 64.976 126.681) (end 64.468 127.189) (width 0.25) (layer B.Cu) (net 28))
 (segment (start 64.976 118.229685) (end 64.976 118.807) (width 0.25) (layer B.Cu) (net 28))
 (segment (start 65.103 118.102685) (end 64.976 118.229685) (width 0.25) (layer B.Cu) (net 28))
 (segment (start 65.103 117.537) (end 65.103 118.102685) (width 0.25) (layer B.Cu) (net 28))
 (segment (start 64.976 126.681) (end 64.976 118.807) (width 0.25) (layer B.Cu) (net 28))
 (segment (start 64.976 118.807) (end 64.976 118.299) (width 0.25) (layer B.Cu) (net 28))
 (segment (start 59.134 135.003919) (end 60.979919 133.158) (width 0.25) (layer F.Cu) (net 20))
 (segment (start 59.134 136.206) (end 59.134 135.003919) (width 0.25) (layer F.Cu) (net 20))
 (segment (start 60.979919 133.158) (end 61.674 133.158) (width 0.25) (layer F.Cu) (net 20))
 (segment (start 62.725 132.107) (end 62.725 129.9) (width 0.25) (layer F.Cu) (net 20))
 (segment (start 61.674 133.158) (end 62.725 132.107) (width 0.25) (layer F.Cu) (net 20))
 (segment (start 80.346 111.17) (end 81.25 111.17) (width 0.25) (layer F.Cu) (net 20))
 (segment (start 62.725 129.05) (end 65.664 126.111) (width 0.25) (layer F.Cu) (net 20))
 (segment (start 62.725 129.9) (end 62.725 129.05) (width 0.25) (layer F.Cu) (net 20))
 (segment (start 65.664 126.111) (end 72.771 126.111) (width 0.25) (layer F.Cu) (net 20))
 (segment (start 72.771 126.111) (end 73.787 125.095) (width 0.25) (layer F.Cu) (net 20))
 (segment (start 73.787 125.095) (end 73.787 117.094) (width 0.25) (layer F.Cu) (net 20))
 (segment (start 79.711 111.17) (end 81.25 111.17) (width 0.25) (layer F.Cu) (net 20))
 (segment (start 73.787 117.094) (end 79.711 111.17) (width 0.25) (layer F.Cu) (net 20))
 (segment (start 63.375 130.75) (end 63.375 129.9) (width 0.25) (layer F.Cu) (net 21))
 (segment (start 63.375 133.302919) (end 63.375 130.75) (width 0.25) (layer F.Cu) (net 21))
 (segment (start 61.674 135.003919) (end 63.375 133.302919) (width 0.25) (layer F.Cu) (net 21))
 (segment (start 61.674 136.206) (end 61.674 135.003919) (width 0.25) (layer F.Cu) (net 21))
 (segment (start 63.375 129.05) (end 65.806 126.619) (width 0.25) (layer F.Cu) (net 21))
 (segment (start 63.375 129.9) (end 63.375 129.05) (width 0.25) (layer F.Cu) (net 21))
 (segment (start 65.806 126.619) (end 73.025 126.619) (width 0.25) (layer F.Cu) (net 21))
 (segment (start 73.025 126.619) (end 74.295 125.349) (width 0.25) (layer F.Cu) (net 21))
 (segment (start 74.295 125.349) (end 74.295 117.475) (width 0.25) (layer F.Cu) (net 21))
 (segment (start 79.33 112.44) (end 81.25 112.44) (width 0.25) (layer F.Cu) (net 21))
 (segment (start 74.295 117.475) (end 79.33 112.44) (width 0.25) (layer F.Cu) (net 21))
 (segment (start 64.025 130.75) (end 64.025 129.9) (width 0.25) (layer F.Cu) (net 22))
 (segment (start 64.025 134.814919) (end 64.025 130.75) (width 0.25) (layer F.Cu) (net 22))
 (segment (start 64.214 135.003919) (end 64.025 134.814919) (width 0.25) (layer F.Cu) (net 22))
 (segment (start 64.214 136.206) (end 64.214 135.003919) (width 0.25) (layer F.Cu) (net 22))
 (segment (start 64.025 129.05) (end 65.948 127.127) (width 0.25) (layer F.Cu) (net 22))
 (segment (start 64.025 129.9) (end 64.025 129.05) (width 0.25) (layer F.Cu) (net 22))
 (segment (start 65.948 127.127) (end 73.279 127.127) (width 0.25) (layer F.Cu) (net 22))
 (segment (start 73.279 127.127) (end 74.93 125.476) (width 0.25) (layer F.Cu) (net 22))
 (segment (start 74.93 125.476) (end 74.93 117.729) (width 0.25) (layer F.Cu) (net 22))
 (segment (start 78.949 113.71) (end 81.25 113.71) (width 0.25) (layer F.Cu) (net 22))
 (segment (start 74.93 117.729) (end 78.949 113.71) (width 0.25) (layer F.Cu) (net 22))
 (segment (start 66.754 135.003919) (end 65.797081 134.047) (width 0.25) (layer F.Cu) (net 23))
 (segment (start 66.754 136.206) (end 66.754 135.003919) (width 0.25) (layer F.Cu) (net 23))
 (segment (start 64.675 132.73) (end 64.675 131.126) (width 0.25) (layer F.Cu) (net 23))
 (segment (start 65.797081 133.852081) (end 64.675 132.73) (width 0.25) (layer F.Cu) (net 23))
 (segment (start 65.797081 134.047) (end 65.797081 133.852081) (width 0.25) (layer F.Cu) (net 23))
 (segment (start 64.675 129.9) (end 64.675 131.126) (width 0.25) (layer F.Cu) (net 23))
 (segment (start 64.675 129.05) (end 66.09 127.635) (width 0.25) (layer F.Cu) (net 23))
 (segment (start 64.675 129.9) (end 64.675 129.05) (width 0.25) (layer F.Cu) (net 23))
 (segment (start 66.09 127.635) (end 73.533 127.635) (width 0.25) (layer F.Cu) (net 23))
 (segment (start 73.533 127.635) (end 75.438 125.73) (width 0.25) (layer F.Cu) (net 23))
 (segment (start 75.438 125.73) (end 75.438 118.364) (width 0.25) (layer F.Cu) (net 23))
 (segment (start 78.822 114.98) (end 81.25 114.98) (width 0.25) (layer F.Cu) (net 23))
 (segment (start 75.438 118.364) (end 78.822 114.98) (width 0.25) (layer F.Cu) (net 23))
 (segment (start 65.325 132.237) (end 65.325 129.9) (width 0.25) (layer F.Cu) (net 24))
 (segment (start 69.294 136.206) (end 65.325 132.237) (width 0.25) (layer F.Cu) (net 24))
 (segment (start 65.325 129.05) (end 66.232 128.143) (width 0.25) (layer F.Cu) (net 24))
 (segment (start 65.325 129.9) (end 65.325 129.05) (width 0.25) (layer F.Cu) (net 24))
 (segment (start 66.232 128.143) (end 73.787 128.143) (width 0.25) (layer F.Cu) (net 24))
 (segment (start 73.787 128.143) (end 75.946 125.984) (width 0.25) (layer F.Cu) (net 24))
 (segment (start 75.946 125.984) (end 75.946 118.872) (width 0.25) (layer F.Cu) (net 24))
 (segment (start 78.568 116.25) (end 81.25 116.25) (width 0.25) (layer F.Cu) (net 24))
 (segment (start 75.946 118.872) (end 78.568 116.25) (width 0.25) (layer F.Cu) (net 24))
 (segment (start 65.975 129.9) (end 65.975 131.744) (width 0.25) (layer F.Cu) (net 25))
 (segment (start 65.975 131.744) (end 68.913 134.682) (width 0.25) (layer F.Cu) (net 25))
 (segment (start 70.31 134.682) (end 71.834 136.206) (width 0.25) (layer F.Cu) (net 25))
 (segment (start 68.913 134.682) (end 70.31 134.682) (width 0.25) (layer F.Cu) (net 25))
 (segment (start 78.441 117.52) (end 81.25 117.52) (width 0.25) (layer F.Cu) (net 25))
 (segment (start 65.975 129.9) (end 65.975 129.05) (width 0.25) (layer F.Cu) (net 25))
 (segment (start 66.374 128.651) (end 74.041 128.651) (width 0.25) (layer F.Cu) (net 25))
 (segment (start 74.041 128.651) (end 76.454 126.238) (width 0.25) (layer F.Cu) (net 25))
 (segment (start 76.454 126.238) (end 76.454 119.507) (width 0.25) (layer F.Cu) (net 25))
 (segment (start 65.975 129.05) (end 66.374 128.651) (width 0.25) (layer F.Cu) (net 25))
 (segment (start 76.454 119.507) (end 78.441 117.52) (width 0.25) (layer F.Cu) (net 25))
 (segment (start 69.802 114.87) (end 69.802 117.646) (width 0.25) (layer F.Cu) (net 15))
 (segment (start 68.532 113.6) (end 69.802 114.87) (width 0.25) (layer F.Cu) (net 15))
 (segment (start 63.849 116.1775) (end 63.849 114.092) (width 0.25) (layer F.Cu) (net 15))
 (segment (start 64.341 113.6) (end 68.532 113.6) (width 0.25) (layer F.Cu) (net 15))
 (segment (start 63.849 114.092) (end 64.341 113.6) (width 0.25) (layer F.Cu) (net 15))
 (segment (start 105.83 116.25) (end 106 116.08) (width 0.25) (layer F.Cu) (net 19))
 (segment (start 98.75 116.25) (end 105.83 116.25) (width 0.4) (layer F.Cu) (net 19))
 (segment (start 98.75 112.44) (end 102.444 112.44) (width 0.4) (layer F.Cu) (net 18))
 (segment (start 103.544 113.54) (end 106 113.54) (width 0.4) (layer F.Cu) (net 18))
 (segment (start 102.444 112.44) (end 103.544 113.54) (width 0.4) (layer F.Cu) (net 18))
 (segment (start 105.83 111.17) (end 106 111) (width 0.25) (layer F.Cu) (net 17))
 (segment (start 98.75 111.17) (end 105.83 111.17) (width 0.4) (layer F.Cu) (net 17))
 (segment (start 98.75 109.9) (end 102.825 109.9) (width 0.4) (layer F.Cu) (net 16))
 (segment (start 104.265 108.46) (end 106 108.46) (width 0.4) (layer F.Cu) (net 16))
 (segment (start 102.825 109.9) (end 104.265 108.46) (width 0.4) (layer F.Cu) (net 16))
 (segment (start 102.03 122.6) (end 98.75 122.6) (width 0.4) (layer F.Cu) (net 14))
 (segment (start 102.873 124.118) (end 102.873 123.443) (width 0.4) (layer F.Cu) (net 14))
 (segment (start 102.873 123.443) (end 102.03 122.6) (width 0.4) (layer F.Cu) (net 14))
 (segment (start 102.873 126.168) (end 104.873 126.168) (width 0.4) (layer F.Cu) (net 13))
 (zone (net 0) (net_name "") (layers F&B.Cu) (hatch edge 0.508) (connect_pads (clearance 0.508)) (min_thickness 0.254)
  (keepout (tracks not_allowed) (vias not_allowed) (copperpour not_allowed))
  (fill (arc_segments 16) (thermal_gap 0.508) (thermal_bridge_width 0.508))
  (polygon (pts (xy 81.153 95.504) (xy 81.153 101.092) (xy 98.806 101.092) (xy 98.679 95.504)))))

